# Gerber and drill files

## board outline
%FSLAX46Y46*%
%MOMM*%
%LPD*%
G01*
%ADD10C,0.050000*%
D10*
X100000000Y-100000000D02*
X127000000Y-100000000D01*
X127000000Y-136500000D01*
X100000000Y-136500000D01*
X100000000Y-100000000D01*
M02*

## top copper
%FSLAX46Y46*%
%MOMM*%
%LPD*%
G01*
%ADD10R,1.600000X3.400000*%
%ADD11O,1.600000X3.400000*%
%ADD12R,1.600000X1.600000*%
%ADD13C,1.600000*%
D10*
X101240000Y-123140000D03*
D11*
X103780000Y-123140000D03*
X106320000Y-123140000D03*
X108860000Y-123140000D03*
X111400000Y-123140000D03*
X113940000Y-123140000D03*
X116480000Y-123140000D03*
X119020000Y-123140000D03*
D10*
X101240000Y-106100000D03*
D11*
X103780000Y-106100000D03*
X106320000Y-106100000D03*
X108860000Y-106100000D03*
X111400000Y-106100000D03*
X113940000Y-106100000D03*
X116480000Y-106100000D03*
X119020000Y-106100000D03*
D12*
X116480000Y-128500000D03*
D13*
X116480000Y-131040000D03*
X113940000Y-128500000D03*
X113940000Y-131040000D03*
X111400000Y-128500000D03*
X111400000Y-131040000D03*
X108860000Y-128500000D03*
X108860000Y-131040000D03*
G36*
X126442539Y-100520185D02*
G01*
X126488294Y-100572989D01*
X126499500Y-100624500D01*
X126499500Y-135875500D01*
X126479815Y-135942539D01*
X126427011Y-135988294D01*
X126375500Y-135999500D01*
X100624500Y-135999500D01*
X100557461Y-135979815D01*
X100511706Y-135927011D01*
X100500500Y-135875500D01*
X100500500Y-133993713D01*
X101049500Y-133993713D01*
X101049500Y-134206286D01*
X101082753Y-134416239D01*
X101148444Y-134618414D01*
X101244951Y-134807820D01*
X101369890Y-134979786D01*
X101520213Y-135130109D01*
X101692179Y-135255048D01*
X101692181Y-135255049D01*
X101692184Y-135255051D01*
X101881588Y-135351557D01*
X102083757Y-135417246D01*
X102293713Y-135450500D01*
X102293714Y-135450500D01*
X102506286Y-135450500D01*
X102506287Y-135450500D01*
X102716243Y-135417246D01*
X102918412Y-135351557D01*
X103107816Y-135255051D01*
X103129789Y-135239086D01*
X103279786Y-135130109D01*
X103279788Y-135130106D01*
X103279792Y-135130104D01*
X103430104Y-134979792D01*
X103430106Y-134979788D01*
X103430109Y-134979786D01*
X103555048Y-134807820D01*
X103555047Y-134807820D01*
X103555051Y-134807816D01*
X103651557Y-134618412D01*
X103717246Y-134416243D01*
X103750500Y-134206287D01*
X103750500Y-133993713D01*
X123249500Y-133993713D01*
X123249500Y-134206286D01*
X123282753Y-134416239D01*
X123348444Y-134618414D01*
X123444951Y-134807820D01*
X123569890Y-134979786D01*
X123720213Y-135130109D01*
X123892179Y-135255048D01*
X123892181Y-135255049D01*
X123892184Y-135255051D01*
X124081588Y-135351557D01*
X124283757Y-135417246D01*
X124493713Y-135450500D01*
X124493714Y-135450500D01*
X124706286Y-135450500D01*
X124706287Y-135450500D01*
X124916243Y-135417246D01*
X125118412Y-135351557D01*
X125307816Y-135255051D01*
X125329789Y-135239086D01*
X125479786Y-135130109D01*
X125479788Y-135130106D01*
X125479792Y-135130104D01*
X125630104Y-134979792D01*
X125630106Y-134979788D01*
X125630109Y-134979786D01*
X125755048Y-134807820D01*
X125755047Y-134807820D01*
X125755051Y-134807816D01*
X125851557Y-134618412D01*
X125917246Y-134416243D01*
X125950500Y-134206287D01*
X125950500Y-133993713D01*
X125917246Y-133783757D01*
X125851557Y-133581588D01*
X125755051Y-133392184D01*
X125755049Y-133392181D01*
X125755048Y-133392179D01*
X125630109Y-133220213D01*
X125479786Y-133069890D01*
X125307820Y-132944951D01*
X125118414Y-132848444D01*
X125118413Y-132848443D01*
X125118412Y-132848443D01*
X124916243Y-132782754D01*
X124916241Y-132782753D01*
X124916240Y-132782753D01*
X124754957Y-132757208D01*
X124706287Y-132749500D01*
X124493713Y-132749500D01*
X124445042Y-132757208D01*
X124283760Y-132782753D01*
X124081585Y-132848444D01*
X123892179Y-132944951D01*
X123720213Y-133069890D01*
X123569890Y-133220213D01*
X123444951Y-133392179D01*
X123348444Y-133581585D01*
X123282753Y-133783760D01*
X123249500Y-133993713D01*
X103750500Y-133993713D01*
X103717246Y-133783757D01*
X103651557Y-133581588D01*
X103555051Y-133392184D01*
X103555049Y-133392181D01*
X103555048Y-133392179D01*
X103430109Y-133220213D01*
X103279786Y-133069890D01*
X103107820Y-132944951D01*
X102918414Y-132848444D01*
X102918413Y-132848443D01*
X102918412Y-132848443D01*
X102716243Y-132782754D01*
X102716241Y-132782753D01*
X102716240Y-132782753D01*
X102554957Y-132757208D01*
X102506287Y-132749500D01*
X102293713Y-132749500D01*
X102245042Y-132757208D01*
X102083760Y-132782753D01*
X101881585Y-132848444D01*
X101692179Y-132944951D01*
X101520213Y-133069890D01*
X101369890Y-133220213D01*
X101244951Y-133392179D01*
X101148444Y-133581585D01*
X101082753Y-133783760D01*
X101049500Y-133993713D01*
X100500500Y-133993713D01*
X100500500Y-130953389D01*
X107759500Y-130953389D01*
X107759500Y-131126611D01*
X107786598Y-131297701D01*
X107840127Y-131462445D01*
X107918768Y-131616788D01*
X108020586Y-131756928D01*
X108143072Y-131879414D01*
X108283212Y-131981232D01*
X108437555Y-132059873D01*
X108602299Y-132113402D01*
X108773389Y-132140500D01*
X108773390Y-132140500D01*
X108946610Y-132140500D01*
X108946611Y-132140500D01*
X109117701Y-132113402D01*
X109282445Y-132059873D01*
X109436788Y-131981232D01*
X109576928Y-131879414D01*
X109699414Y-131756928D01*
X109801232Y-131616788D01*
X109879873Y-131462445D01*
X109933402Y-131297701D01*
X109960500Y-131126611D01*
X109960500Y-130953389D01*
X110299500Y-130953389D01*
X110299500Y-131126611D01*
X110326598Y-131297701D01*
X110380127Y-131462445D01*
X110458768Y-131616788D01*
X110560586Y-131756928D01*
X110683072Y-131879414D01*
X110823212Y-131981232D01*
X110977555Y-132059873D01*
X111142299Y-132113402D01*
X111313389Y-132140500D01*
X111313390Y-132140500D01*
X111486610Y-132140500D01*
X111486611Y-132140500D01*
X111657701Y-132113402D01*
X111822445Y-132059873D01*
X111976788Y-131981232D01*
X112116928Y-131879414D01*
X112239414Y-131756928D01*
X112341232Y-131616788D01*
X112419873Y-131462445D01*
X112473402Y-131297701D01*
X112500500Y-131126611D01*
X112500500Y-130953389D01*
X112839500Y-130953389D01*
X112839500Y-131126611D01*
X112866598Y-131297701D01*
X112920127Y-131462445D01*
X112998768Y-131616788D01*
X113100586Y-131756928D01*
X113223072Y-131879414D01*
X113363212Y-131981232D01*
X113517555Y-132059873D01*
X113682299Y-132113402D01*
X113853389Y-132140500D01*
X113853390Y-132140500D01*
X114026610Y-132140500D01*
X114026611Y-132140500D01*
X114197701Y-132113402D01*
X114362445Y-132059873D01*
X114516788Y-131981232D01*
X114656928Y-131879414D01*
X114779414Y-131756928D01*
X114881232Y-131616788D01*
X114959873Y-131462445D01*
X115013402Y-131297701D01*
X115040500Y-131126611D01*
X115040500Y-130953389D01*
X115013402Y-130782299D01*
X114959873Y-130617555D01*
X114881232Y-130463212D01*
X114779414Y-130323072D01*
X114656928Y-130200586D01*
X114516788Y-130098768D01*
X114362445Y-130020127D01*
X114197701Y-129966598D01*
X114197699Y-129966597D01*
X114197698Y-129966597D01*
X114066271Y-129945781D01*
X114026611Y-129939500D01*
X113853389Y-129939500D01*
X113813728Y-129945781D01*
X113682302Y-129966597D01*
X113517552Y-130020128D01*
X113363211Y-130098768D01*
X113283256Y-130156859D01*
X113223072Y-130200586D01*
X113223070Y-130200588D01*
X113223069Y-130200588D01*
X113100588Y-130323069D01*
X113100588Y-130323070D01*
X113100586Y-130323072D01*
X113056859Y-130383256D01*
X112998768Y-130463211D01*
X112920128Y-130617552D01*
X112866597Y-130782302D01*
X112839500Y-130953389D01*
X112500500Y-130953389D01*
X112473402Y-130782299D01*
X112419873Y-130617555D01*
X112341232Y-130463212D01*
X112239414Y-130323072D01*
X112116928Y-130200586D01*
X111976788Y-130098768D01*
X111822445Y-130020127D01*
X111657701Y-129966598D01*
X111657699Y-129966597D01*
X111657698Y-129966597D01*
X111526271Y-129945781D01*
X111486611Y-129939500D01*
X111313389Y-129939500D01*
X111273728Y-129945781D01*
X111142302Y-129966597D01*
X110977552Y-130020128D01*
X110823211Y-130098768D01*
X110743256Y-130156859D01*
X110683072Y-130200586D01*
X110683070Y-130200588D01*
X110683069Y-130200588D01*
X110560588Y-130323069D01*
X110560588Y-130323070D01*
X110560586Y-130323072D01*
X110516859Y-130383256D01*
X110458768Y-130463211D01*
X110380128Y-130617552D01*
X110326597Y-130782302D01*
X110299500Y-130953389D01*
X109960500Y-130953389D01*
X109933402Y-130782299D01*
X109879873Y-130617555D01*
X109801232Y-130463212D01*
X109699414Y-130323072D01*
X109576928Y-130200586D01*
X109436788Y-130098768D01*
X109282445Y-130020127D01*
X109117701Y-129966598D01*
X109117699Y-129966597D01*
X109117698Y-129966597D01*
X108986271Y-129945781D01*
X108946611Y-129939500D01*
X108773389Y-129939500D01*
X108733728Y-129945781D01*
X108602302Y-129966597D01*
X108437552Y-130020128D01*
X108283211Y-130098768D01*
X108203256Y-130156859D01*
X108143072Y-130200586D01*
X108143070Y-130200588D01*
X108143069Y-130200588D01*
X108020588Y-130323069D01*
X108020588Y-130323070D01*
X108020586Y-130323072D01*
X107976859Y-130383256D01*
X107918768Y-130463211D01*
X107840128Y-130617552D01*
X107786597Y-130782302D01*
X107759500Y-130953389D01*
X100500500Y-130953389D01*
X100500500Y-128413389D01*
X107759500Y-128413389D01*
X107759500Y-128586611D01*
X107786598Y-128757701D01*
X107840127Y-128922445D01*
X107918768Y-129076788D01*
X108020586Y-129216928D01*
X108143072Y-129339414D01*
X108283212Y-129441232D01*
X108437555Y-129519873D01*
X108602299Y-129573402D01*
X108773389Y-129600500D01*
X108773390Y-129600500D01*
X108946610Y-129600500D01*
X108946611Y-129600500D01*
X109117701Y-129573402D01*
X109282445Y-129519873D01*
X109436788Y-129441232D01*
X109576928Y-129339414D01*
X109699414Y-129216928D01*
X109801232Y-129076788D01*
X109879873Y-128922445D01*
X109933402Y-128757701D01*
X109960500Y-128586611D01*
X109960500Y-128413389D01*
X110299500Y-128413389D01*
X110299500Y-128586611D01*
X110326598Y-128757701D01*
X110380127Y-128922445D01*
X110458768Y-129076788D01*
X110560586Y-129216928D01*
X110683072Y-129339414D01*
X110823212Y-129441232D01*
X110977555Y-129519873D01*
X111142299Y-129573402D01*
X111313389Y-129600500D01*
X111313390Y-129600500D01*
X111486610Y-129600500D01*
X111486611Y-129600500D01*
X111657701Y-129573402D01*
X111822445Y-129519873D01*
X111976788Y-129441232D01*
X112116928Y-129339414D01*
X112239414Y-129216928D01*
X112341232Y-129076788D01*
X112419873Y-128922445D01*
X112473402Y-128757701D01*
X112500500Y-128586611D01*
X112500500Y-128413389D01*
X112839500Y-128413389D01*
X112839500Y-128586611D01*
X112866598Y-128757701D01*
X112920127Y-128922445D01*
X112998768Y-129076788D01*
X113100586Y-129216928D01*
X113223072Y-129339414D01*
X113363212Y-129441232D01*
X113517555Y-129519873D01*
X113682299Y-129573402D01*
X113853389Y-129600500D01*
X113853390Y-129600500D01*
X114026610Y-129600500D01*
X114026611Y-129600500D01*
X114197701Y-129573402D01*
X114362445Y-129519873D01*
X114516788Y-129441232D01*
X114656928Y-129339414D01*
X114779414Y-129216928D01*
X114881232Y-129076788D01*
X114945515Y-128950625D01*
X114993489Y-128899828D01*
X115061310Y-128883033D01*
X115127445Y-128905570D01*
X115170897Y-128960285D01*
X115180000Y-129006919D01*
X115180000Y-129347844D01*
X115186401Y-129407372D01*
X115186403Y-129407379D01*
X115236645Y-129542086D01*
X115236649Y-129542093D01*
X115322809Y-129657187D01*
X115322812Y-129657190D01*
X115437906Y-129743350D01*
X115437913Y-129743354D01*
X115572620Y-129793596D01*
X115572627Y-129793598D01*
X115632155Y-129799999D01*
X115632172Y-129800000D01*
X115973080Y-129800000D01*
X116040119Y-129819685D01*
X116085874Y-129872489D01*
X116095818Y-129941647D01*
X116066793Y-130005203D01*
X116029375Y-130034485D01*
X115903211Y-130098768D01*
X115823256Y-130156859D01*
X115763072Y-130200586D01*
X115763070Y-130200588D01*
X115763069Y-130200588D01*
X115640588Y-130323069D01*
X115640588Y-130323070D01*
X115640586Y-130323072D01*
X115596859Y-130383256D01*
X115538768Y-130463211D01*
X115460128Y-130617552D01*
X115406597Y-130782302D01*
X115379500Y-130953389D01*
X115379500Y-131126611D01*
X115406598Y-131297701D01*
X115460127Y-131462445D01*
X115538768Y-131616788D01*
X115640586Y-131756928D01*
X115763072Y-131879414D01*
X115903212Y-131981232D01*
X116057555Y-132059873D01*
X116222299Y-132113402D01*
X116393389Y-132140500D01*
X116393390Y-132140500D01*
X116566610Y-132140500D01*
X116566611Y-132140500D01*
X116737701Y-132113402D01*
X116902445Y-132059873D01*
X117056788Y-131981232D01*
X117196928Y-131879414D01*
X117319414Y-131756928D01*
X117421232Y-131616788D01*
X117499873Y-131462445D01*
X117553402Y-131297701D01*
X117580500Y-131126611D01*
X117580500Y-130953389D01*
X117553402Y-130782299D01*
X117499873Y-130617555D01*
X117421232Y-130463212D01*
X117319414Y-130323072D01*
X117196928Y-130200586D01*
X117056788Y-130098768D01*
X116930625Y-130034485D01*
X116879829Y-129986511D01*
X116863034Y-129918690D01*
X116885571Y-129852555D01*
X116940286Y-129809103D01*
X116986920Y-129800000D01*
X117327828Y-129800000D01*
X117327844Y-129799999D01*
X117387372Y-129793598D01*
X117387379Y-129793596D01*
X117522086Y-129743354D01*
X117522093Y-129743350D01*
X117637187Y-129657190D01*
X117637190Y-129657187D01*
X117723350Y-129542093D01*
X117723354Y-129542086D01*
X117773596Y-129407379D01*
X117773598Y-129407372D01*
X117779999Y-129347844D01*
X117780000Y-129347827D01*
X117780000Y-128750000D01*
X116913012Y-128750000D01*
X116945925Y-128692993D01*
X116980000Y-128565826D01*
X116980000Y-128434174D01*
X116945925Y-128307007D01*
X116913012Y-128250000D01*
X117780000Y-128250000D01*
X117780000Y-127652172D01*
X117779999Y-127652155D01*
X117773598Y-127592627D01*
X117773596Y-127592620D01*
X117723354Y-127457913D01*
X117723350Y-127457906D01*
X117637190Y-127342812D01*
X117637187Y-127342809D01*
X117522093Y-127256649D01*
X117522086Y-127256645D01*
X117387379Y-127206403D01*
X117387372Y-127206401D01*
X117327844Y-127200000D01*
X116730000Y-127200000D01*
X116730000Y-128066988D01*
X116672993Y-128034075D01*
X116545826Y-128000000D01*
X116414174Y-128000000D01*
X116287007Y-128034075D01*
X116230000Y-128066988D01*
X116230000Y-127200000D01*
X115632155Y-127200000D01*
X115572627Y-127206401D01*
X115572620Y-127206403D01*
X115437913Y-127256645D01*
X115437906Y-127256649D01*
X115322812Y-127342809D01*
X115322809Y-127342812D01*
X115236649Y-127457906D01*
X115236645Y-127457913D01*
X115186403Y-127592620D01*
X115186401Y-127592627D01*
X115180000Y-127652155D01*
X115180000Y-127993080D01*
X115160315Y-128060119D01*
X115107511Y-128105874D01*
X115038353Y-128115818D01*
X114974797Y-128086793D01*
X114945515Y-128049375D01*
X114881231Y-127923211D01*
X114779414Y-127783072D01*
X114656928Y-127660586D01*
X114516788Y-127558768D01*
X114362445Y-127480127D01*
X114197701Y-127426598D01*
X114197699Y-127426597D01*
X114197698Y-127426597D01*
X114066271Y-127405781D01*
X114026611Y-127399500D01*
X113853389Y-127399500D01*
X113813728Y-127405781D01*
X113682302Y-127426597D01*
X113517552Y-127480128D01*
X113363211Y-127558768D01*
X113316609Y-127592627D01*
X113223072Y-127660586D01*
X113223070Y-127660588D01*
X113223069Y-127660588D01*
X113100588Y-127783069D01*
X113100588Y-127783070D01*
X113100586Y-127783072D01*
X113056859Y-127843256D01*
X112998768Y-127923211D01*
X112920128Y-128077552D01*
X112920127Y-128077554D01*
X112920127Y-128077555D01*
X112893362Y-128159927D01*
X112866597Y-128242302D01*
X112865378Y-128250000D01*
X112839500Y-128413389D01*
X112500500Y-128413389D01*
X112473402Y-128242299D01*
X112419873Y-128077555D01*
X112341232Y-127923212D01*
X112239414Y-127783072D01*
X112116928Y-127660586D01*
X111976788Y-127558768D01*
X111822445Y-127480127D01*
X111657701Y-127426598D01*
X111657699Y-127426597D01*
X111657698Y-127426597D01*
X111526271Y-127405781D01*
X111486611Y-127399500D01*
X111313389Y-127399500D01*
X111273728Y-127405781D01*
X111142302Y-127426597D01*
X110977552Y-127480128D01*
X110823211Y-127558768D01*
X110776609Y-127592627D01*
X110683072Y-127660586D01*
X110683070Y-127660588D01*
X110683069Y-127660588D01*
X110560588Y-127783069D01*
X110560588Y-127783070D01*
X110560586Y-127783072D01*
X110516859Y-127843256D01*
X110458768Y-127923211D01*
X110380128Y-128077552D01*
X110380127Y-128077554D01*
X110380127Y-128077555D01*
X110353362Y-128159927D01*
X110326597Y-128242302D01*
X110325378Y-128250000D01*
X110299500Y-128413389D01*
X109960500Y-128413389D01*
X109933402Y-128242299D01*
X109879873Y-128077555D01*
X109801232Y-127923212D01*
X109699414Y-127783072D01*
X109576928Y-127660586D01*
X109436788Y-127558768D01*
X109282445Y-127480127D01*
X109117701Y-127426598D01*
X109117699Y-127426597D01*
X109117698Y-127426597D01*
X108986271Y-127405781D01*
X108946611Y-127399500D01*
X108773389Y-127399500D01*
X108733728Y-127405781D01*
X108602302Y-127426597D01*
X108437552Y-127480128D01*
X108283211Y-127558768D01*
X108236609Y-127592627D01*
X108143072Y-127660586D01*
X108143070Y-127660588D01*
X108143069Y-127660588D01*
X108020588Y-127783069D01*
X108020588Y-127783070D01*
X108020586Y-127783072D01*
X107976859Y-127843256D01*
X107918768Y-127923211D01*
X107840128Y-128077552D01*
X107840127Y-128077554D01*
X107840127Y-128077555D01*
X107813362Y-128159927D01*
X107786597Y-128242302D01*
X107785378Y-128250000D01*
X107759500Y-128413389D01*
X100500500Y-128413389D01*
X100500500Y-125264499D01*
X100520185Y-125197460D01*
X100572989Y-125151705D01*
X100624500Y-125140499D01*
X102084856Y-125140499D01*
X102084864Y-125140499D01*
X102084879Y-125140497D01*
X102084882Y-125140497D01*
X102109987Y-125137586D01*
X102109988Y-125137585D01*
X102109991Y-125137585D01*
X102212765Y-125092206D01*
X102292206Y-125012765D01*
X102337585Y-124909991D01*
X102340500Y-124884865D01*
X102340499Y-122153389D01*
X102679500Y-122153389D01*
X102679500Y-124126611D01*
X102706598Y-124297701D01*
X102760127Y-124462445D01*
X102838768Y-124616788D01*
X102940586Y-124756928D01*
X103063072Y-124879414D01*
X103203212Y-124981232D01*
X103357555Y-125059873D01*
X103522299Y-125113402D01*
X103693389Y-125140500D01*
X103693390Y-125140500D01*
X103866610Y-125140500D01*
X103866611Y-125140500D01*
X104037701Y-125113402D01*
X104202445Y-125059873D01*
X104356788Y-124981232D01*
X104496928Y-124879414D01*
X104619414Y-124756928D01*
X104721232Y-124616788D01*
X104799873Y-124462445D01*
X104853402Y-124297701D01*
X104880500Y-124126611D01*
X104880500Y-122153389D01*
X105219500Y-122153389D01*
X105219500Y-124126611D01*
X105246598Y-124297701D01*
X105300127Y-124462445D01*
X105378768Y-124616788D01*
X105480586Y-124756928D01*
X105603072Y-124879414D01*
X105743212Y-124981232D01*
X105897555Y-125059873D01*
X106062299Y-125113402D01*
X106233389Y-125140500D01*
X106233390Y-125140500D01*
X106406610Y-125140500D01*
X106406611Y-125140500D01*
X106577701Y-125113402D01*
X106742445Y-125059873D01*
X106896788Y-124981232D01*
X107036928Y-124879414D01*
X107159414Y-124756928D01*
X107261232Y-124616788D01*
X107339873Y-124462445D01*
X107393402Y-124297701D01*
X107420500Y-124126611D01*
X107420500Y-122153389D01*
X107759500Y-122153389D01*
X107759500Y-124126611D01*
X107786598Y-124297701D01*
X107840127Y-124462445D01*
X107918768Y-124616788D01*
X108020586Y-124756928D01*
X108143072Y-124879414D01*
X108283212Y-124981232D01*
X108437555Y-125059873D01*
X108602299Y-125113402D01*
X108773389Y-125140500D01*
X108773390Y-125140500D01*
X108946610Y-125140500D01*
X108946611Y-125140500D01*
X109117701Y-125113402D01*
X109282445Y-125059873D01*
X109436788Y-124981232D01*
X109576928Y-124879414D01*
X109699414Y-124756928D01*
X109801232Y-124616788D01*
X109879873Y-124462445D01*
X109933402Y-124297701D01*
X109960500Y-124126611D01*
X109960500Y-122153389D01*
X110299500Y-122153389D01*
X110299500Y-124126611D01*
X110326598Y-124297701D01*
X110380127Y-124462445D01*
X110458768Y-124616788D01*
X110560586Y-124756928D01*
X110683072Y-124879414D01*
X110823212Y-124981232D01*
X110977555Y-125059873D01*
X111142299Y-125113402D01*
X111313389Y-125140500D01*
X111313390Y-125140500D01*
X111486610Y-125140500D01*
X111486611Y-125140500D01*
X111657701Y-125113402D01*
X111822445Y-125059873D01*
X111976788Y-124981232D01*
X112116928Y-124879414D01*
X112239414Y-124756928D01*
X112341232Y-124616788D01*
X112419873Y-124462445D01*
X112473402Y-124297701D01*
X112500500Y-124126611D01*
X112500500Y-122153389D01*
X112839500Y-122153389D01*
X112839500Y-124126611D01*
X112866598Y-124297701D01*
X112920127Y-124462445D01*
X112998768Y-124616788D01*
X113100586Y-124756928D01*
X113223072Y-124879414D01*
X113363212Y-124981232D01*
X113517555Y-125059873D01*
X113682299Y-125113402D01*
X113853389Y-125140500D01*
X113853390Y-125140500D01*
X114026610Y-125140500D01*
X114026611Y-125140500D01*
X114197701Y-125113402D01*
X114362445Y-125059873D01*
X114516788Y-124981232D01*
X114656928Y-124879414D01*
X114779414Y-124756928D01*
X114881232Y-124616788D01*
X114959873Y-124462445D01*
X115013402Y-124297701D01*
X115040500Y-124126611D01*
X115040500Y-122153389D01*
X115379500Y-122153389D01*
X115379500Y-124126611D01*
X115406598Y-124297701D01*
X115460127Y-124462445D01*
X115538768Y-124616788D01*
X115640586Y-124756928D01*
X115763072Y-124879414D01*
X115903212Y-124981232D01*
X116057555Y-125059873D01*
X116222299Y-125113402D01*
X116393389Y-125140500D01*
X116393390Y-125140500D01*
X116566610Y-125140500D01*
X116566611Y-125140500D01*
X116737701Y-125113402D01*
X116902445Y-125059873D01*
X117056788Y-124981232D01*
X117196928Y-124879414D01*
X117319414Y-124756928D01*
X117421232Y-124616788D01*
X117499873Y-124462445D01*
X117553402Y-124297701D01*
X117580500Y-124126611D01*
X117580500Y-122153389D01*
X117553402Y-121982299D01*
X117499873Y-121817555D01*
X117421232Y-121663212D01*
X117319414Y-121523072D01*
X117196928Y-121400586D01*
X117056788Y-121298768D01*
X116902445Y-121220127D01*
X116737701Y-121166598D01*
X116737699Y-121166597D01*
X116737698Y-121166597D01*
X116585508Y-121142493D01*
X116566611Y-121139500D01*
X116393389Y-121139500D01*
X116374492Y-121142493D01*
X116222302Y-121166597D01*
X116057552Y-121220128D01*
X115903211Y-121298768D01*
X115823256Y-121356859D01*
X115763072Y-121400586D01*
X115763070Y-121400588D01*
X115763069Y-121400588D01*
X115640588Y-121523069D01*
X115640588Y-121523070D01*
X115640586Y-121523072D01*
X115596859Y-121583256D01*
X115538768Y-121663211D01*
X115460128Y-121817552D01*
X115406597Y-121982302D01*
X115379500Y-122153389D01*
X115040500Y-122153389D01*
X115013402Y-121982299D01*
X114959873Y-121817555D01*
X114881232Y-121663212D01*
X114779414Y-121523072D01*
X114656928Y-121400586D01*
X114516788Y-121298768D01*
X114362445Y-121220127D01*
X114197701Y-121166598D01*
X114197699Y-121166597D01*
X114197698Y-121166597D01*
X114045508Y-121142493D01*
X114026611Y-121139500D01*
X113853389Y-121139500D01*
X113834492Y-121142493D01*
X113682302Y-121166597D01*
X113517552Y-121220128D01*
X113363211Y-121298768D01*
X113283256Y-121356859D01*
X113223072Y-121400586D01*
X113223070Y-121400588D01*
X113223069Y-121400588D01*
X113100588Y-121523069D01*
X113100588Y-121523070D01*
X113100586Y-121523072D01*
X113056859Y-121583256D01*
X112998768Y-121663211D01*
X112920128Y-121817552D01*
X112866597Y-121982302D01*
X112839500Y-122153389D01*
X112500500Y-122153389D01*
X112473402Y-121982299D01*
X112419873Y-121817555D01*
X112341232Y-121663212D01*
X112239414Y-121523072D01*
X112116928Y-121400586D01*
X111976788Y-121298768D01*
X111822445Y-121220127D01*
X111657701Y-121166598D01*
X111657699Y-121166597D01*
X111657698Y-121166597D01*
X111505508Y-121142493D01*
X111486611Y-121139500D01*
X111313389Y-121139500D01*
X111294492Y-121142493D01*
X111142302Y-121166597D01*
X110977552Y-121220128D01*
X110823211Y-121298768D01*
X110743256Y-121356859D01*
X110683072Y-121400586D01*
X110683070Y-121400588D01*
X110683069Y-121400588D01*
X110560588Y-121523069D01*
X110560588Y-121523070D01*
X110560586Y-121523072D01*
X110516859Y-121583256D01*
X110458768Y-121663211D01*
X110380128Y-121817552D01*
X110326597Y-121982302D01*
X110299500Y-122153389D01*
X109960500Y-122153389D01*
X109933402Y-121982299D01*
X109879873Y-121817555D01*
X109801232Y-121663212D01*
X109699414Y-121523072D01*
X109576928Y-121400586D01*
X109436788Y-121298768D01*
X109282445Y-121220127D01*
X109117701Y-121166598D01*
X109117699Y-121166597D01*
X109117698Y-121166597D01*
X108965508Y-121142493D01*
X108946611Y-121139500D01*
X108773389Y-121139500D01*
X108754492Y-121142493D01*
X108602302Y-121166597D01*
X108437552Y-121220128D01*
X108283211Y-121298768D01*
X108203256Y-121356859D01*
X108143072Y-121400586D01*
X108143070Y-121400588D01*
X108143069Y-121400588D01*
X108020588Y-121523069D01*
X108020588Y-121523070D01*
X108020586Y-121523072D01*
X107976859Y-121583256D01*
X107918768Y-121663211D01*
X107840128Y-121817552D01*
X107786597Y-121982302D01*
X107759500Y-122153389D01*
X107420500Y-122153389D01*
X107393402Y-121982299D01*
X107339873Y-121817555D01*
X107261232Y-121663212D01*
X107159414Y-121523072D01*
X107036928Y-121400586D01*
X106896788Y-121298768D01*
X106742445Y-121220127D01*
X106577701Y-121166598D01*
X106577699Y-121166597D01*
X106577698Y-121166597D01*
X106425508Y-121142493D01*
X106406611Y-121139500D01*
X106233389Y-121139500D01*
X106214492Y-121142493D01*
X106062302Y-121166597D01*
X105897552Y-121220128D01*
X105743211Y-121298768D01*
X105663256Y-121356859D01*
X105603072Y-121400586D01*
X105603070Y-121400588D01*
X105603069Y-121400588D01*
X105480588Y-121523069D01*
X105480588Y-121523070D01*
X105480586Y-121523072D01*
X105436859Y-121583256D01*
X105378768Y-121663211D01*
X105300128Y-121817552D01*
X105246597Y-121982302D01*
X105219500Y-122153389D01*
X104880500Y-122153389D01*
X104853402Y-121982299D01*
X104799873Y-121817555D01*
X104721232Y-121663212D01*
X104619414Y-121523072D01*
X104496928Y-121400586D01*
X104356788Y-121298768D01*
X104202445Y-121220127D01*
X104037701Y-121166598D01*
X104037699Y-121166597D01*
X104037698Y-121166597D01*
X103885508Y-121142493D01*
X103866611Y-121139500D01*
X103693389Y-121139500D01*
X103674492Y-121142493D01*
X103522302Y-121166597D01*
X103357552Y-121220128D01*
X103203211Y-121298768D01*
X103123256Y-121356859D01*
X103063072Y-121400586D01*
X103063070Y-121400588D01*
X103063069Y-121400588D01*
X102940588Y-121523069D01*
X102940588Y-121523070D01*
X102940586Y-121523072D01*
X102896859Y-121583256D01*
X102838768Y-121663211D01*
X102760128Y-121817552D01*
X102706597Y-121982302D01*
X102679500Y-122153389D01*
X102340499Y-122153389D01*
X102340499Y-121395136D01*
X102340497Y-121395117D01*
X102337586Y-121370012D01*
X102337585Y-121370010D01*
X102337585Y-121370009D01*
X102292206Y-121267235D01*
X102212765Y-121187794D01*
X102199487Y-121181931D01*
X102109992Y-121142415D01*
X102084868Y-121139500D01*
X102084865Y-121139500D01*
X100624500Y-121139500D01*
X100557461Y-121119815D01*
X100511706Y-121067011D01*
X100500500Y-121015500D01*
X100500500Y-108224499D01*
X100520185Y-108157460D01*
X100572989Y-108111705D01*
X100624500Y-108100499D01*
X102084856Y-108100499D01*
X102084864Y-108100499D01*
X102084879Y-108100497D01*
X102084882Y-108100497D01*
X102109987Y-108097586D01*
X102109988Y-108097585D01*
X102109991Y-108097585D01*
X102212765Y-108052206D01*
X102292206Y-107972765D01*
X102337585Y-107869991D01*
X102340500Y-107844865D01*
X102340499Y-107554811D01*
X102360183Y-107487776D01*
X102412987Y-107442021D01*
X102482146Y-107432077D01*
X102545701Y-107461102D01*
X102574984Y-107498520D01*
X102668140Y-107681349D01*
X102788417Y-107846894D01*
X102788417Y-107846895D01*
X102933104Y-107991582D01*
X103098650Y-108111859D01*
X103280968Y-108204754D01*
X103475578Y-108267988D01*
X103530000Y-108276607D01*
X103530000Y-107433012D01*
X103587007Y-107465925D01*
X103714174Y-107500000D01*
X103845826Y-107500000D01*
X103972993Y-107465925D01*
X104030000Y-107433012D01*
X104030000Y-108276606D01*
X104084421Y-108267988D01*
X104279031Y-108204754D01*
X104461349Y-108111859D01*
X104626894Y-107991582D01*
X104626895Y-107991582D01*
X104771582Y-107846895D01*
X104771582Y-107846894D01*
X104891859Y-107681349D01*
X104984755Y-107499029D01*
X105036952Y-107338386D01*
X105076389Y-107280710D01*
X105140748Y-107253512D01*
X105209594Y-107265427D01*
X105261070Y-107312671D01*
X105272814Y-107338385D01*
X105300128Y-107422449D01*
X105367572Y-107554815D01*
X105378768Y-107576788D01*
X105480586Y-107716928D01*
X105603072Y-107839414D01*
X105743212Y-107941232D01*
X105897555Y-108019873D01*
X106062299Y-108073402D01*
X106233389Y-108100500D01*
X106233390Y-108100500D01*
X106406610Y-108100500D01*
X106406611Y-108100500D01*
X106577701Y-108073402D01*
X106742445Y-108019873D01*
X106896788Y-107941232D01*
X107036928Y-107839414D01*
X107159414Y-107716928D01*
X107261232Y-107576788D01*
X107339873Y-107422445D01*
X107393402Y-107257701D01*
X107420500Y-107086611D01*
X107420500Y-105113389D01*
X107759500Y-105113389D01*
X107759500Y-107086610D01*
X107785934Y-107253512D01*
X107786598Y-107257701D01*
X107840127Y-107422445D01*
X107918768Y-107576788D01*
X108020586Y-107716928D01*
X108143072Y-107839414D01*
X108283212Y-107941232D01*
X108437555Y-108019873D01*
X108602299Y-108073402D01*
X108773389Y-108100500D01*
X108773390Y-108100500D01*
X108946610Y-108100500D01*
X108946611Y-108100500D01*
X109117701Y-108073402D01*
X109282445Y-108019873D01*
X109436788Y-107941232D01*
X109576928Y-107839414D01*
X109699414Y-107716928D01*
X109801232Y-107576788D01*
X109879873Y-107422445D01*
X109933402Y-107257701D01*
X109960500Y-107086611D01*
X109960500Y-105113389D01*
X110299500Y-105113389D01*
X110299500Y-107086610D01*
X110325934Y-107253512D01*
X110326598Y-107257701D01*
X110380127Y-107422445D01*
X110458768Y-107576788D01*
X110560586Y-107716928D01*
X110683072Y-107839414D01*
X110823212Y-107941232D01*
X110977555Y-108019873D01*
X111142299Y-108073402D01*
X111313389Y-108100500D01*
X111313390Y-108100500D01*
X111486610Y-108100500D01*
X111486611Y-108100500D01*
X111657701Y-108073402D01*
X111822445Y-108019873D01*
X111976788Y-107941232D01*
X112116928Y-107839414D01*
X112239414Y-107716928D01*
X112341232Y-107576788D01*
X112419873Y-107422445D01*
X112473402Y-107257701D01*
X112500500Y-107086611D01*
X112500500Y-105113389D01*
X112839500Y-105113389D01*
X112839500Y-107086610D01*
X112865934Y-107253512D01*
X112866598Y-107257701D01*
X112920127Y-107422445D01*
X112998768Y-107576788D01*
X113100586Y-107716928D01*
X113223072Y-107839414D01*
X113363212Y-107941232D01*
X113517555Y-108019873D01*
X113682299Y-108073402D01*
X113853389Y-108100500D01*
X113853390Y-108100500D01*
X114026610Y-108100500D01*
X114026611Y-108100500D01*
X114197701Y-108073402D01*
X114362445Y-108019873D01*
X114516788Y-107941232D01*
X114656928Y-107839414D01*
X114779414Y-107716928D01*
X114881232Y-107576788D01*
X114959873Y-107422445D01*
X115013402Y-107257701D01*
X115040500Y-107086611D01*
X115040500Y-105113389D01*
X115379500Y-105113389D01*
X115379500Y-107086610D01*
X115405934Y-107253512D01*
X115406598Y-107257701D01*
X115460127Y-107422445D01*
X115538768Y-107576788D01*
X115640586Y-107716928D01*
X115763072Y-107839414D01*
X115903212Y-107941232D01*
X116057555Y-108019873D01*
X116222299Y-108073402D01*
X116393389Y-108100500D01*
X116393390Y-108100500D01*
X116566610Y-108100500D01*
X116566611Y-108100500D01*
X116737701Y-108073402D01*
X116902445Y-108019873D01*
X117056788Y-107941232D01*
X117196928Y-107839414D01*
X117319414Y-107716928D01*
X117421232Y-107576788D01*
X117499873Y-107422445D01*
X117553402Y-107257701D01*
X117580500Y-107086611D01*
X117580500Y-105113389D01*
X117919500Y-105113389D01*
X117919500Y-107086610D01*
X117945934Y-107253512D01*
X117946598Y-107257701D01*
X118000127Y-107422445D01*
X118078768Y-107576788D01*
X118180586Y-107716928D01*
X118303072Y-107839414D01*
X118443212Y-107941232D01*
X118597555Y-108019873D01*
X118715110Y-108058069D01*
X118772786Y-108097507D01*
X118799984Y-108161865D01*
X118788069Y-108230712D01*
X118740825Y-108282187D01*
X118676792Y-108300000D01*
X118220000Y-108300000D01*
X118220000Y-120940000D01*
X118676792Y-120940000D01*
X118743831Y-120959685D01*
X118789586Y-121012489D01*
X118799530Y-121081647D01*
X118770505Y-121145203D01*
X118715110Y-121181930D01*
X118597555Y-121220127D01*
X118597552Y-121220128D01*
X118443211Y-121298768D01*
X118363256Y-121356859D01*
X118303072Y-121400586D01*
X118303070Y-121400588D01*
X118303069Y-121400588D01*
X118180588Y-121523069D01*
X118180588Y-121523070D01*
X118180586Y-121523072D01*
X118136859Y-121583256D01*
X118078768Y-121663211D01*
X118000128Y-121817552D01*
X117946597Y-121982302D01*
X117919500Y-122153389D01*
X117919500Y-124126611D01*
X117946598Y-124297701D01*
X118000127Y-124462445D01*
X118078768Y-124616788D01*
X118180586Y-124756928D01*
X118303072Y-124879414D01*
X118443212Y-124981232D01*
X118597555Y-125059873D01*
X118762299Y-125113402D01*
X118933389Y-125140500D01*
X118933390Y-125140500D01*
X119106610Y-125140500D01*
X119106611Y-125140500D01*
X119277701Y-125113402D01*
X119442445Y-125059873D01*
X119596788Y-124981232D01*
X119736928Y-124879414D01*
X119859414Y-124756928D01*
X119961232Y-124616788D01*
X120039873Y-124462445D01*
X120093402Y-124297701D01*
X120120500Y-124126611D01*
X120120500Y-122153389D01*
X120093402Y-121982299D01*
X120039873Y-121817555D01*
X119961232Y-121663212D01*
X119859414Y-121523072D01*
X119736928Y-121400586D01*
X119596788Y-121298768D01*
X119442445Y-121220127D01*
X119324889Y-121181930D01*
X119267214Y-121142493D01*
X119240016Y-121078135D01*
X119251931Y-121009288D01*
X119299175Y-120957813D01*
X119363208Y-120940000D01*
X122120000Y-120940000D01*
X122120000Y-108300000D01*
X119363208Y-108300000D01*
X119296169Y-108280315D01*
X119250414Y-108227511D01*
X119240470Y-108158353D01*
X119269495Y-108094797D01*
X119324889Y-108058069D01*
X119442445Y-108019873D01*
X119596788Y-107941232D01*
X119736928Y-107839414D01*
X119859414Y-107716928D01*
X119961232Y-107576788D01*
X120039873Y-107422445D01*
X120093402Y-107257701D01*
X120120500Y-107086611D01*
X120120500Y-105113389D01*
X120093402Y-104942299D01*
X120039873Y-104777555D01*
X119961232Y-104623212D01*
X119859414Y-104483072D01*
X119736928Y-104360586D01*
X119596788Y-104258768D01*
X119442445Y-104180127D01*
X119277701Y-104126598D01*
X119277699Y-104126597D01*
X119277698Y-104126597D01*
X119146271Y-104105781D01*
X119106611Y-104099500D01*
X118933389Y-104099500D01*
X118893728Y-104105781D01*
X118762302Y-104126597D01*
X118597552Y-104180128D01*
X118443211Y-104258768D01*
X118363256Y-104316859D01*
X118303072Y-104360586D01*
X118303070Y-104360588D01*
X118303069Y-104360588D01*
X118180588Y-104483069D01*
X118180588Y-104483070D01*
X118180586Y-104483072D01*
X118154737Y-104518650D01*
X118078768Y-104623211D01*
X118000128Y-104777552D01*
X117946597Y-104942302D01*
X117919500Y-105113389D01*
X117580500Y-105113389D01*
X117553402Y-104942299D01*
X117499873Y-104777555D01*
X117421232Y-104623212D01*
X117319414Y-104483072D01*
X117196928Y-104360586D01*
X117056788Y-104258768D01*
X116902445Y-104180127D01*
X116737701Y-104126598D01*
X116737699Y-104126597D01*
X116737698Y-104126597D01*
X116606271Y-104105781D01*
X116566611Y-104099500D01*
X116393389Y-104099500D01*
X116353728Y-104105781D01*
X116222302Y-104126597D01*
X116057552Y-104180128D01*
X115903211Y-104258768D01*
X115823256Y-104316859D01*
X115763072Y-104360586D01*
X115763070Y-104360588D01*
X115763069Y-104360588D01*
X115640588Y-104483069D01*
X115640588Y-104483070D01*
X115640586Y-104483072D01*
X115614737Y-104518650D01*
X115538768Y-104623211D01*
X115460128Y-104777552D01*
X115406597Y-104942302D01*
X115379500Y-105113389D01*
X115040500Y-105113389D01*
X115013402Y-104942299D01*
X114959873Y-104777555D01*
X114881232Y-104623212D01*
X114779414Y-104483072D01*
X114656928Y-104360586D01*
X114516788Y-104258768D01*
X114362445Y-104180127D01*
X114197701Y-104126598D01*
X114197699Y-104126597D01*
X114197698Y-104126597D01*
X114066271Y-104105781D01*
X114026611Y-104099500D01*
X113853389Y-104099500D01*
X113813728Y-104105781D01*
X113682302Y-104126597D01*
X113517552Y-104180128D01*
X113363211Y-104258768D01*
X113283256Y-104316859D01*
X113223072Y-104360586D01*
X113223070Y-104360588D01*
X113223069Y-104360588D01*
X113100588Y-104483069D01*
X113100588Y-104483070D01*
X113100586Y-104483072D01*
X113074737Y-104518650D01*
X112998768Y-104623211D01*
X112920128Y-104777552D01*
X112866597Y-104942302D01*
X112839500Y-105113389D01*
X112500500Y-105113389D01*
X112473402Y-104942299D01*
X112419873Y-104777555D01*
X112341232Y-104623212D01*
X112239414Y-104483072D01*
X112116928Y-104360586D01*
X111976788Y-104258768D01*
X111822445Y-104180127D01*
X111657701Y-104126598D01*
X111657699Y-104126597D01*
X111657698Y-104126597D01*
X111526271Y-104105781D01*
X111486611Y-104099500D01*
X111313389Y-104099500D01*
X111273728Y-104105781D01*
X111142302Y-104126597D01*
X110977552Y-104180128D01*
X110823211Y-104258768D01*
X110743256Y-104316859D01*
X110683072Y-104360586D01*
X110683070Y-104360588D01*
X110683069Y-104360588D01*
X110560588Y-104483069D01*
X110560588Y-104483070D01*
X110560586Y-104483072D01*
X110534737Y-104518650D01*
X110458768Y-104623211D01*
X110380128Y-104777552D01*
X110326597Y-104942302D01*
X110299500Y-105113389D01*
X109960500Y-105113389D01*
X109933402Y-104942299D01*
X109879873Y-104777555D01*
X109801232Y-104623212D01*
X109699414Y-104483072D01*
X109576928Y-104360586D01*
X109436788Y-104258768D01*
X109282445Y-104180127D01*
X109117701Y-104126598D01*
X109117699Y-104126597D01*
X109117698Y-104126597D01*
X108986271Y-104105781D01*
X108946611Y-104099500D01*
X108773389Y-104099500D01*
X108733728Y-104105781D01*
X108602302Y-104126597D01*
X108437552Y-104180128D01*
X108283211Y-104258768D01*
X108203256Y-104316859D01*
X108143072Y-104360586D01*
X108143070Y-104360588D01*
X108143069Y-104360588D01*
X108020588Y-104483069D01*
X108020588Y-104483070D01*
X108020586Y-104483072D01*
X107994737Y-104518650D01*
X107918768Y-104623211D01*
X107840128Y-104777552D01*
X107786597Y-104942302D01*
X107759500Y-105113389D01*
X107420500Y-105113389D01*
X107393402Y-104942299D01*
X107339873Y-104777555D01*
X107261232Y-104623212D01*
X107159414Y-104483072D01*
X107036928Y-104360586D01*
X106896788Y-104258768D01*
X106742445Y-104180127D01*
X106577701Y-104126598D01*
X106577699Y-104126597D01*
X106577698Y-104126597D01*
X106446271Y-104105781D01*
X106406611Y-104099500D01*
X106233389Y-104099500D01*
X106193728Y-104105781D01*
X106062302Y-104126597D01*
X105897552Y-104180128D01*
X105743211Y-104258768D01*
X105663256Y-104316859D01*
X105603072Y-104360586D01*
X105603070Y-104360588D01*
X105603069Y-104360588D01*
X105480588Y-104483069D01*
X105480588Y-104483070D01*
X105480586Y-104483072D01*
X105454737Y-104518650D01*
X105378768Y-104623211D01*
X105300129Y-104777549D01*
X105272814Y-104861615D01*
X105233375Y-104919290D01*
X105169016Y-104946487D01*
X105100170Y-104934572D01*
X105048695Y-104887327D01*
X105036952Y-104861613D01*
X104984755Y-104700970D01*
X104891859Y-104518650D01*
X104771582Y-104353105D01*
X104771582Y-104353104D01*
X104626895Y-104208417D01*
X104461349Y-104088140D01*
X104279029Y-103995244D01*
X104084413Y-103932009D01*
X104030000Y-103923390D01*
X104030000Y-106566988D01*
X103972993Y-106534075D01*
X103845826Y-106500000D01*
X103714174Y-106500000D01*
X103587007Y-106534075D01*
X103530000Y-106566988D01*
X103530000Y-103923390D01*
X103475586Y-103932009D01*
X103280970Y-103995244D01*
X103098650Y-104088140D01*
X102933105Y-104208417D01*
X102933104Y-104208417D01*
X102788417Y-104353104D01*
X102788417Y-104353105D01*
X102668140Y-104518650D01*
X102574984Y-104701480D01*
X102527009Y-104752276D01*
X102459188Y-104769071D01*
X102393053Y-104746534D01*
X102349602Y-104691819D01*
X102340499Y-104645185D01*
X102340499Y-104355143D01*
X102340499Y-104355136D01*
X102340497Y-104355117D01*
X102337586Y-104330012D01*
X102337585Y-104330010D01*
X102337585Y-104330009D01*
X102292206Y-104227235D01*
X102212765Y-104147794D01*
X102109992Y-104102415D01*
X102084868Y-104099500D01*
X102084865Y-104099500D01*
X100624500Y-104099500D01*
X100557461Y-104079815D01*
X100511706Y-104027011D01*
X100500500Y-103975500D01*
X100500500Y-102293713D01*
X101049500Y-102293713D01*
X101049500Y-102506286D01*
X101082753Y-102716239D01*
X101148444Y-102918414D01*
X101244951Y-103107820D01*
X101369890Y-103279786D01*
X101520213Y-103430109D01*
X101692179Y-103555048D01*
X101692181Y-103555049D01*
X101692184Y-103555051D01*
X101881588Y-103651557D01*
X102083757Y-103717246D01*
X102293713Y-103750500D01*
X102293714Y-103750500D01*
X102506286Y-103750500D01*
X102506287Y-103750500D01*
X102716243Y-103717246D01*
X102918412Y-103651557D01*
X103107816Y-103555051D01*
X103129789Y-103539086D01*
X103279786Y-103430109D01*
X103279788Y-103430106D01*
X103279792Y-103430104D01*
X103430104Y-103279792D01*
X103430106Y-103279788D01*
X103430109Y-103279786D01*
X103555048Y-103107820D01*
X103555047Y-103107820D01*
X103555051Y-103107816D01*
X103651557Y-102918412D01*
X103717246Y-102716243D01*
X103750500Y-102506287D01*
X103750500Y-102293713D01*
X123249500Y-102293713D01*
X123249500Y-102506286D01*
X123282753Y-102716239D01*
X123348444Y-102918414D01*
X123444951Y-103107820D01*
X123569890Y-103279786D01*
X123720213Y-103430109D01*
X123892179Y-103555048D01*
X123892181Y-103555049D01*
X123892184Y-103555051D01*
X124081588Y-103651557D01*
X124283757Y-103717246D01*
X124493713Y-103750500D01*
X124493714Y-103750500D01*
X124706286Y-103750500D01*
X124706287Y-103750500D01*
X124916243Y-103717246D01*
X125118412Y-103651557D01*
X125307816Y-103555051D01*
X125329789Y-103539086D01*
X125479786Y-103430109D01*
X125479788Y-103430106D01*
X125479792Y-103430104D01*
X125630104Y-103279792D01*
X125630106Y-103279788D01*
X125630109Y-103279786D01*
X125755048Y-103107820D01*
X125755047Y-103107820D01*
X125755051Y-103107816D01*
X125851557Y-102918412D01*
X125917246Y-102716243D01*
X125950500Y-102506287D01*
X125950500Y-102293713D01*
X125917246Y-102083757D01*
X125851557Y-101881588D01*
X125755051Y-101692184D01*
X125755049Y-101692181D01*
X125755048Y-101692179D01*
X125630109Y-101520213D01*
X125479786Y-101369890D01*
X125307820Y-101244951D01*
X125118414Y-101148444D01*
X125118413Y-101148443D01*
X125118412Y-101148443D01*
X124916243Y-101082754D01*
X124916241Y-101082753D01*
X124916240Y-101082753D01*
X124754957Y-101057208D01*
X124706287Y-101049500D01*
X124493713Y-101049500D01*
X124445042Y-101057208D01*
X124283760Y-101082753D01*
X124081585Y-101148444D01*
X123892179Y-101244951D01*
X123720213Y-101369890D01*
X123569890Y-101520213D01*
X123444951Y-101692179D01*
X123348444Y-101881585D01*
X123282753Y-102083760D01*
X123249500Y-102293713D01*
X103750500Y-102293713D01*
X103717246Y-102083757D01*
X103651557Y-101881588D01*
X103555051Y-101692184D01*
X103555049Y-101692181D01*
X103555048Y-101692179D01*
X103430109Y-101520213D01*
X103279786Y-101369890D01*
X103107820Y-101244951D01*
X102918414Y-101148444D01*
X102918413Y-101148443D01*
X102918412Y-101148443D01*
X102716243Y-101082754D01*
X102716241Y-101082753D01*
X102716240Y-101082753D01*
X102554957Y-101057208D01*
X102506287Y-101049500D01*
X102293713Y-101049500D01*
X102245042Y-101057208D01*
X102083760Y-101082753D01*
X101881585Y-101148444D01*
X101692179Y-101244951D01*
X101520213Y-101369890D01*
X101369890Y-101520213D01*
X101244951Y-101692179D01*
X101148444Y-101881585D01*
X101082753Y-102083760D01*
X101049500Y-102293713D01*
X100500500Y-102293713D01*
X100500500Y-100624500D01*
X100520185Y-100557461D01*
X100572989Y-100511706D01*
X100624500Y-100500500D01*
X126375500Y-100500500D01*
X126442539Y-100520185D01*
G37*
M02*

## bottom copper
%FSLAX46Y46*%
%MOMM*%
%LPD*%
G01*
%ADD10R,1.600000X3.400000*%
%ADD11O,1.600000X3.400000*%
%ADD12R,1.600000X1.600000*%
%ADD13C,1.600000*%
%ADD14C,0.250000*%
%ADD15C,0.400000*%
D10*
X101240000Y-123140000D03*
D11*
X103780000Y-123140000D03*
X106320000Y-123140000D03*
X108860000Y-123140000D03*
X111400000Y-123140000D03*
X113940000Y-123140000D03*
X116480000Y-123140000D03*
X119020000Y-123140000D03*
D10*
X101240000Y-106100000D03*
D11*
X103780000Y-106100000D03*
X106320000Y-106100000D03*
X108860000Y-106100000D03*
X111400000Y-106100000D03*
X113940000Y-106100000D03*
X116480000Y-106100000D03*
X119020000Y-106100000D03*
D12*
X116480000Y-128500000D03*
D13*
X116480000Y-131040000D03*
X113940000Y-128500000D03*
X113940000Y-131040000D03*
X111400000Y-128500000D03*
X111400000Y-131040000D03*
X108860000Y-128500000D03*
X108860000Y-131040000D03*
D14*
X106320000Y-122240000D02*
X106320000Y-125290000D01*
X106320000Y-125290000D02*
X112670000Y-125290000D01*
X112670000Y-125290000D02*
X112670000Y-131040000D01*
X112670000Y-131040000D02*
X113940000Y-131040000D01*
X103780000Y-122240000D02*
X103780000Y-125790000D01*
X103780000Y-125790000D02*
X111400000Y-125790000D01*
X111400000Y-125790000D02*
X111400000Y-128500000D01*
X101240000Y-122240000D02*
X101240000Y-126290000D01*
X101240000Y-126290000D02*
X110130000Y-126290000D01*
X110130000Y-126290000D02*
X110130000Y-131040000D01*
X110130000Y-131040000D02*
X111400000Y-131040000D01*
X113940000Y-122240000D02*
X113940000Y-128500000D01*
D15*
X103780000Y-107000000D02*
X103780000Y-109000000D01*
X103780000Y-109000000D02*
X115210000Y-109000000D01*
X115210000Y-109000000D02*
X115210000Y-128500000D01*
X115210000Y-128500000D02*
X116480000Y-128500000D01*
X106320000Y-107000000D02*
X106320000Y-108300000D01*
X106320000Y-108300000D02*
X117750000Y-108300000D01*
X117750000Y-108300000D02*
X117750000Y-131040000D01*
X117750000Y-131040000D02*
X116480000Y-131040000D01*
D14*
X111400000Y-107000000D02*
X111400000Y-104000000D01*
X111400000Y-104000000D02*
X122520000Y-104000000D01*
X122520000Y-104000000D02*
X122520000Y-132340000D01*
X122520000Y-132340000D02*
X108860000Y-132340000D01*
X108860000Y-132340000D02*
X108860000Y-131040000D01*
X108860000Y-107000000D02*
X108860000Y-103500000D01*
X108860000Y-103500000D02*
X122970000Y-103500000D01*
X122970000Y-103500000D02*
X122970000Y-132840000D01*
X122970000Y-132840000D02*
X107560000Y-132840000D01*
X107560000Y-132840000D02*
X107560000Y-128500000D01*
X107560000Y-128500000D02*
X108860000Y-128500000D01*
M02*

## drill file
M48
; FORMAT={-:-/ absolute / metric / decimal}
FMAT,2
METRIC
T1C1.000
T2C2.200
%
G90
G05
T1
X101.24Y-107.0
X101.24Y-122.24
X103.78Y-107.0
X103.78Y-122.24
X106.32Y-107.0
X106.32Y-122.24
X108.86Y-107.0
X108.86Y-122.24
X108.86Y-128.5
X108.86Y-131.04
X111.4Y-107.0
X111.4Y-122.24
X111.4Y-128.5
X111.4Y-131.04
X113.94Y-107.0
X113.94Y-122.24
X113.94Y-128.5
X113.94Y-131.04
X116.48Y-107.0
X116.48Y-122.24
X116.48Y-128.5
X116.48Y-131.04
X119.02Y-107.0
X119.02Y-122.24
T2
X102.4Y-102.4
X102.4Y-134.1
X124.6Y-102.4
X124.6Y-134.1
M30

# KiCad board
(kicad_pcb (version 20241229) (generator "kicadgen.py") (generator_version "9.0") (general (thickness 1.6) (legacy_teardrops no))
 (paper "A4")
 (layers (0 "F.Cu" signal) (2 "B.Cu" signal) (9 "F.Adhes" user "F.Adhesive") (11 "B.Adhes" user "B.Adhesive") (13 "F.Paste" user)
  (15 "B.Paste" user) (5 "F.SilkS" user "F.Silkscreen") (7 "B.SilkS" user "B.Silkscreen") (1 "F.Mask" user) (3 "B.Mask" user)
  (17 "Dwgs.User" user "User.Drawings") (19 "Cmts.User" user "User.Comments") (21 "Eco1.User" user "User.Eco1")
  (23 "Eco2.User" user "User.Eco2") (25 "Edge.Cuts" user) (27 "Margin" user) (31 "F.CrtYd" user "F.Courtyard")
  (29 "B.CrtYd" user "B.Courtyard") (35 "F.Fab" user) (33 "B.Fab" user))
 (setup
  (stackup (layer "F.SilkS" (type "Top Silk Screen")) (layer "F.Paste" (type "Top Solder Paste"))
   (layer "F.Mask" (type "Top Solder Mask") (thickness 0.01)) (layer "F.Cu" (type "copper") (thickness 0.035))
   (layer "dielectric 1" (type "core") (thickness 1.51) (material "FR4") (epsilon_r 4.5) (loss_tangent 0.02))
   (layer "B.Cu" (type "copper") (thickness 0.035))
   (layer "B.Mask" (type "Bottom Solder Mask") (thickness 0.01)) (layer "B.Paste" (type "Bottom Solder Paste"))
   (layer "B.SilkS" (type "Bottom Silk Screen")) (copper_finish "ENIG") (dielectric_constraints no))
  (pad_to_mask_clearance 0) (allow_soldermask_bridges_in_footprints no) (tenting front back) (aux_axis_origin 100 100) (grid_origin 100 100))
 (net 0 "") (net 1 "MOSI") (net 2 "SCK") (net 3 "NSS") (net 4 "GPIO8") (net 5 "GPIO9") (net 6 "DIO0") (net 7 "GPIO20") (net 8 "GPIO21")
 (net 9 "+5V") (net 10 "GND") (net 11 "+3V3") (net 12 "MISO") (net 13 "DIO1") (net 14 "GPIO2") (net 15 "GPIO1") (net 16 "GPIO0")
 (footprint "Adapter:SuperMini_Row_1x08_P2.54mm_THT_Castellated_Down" (layer "F.Cu") (at 101.24 122.24)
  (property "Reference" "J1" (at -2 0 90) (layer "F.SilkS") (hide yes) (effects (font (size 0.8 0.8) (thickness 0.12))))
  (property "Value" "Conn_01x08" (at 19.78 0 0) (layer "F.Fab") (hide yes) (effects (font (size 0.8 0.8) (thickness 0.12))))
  (pad "1" thru_hole rect (at 0 0) (size 1.6 3.4) (drill 1 (offset 0 0.9)) (layers "*.Cu" "*.Mask") (remove_unused_layers no) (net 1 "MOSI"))
  (pad "2" thru_hole oval (at 2.54 0) (size 1.6 3.4) (drill 1 (offset 0 0.9)) (layers "*.Cu" "*.Mask") (remove_unused_layers no)
   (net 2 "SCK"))
  (pad "3" thru_hole oval (at 5.08 0) (size 1.6 3.4) (drill 1 (offset 0 0.9)) (layers "*.Cu" "*.Mask") (remove_unused_layers no)
   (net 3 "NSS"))
  (pad "4" thru_hole oval (at 7.62 0) (size 1.6 3.4) (drill 1 (offset 0 0.9)) (layers "*.Cu" "*.Mask") (remove_unused_layers no)
   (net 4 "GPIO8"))
  (pad "5" thru_hole oval (at 10.16 0) (size 1.6 3.4) (drill 1 (offset 0 0.9)) (layers "*.Cu" "*.Mask") (remove_unused_layers no)
   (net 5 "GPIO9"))
  (pad "6" thru_hole oval (at 12.7 0) (size 1.6 3.4) (drill 1 (offset 0 0.9)) (layers "*.Cu" "*.Mask") (remove_unused_layers no)
   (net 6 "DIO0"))
  (pad "7" thru_hole oval (at 15.24 0) (size 1.6 3.4) (drill 1 (offset 0 0.9)) (layers "*.Cu" "*.Mask") (remove_unused_layers no)
   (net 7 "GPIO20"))
  (pad "8" thru_hole oval (at 17.78 0) (size 1.6 3.4) (drill 1 (offset 0 0.9)) (layers "*.Cu" "*.Mask") (remove_unused_layers no)
   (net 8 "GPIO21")))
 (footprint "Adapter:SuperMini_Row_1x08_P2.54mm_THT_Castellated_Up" (layer "F.Cu") (at 101.24 107)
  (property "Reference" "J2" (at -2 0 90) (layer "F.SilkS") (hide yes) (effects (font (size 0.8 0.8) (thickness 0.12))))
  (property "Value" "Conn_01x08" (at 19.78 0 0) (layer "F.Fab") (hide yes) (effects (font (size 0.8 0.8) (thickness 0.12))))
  (pad "1" thru_hole rect (at 0 0) (size 1.6 3.4) (drill 1 (offset 0 -0.9)) (layers "*.Cu" "*.Mask") (remove_unused_layers no) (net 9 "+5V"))
  (pad "2" thru_hole oval (at 2.54 0) (size 1.6 3.4) (drill 1 (offset 0 -0.9)) (layers "*.Cu" "*.Mask") (remove_unused_layers no)
   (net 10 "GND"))
  (pad "3" thru_hole oval (at 5.08 0) (size 1.6 3.4) (drill 1 (offset 0 -0.9)) (layers "*.Cu" "*.Mask") (remove_unused_layers no)
   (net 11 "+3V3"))
  (pad "4" thru_hole oval (at 7.62 0) (size 1.6 3.4) (drill 1 (offset 0 -0.9)) (layers "*.Cu" "*.Mask") (remove_unused_layers no)
   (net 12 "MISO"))
  (pad "5" thru_hole oval (at 10.16 0) (size 1.6 3.4) (drill 1 (offset 0 -0.9)) (layers "*.Cu" "*.Mask") (remove_unused_layers no)
   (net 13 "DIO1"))
  (pad "6" thru_hole oval (at 12.7 0) (size 1.6 3.4) (drill 1 (offset 0 -0.9)) (layers "*.Cu" "*.Mask") (remove_unused_layers no)
   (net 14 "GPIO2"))
  (pad "7" thru_hole oval (at 15.24 0) (size 1.6 3.4) (drill 1 (offset 0 -0.9)) (layers "*.Cu" "*.Mask") (remove_unused_layers no)
   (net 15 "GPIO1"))
  (pad "8" thru_hole oval (at 17.78 0) (size 1.6 3.4) (drill 1 (offset 0 -0.9)) (layers "*.Cu" "*.Mask") (remove_unused_layers no)
   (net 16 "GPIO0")))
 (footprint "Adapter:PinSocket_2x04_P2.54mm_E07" (layer "F.Cu") (at 116.48 128.5)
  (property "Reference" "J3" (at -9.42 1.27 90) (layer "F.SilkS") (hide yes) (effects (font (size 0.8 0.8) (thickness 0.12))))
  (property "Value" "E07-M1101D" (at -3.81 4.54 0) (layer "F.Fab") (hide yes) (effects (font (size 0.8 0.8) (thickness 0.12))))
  (pad "1" thru_hole rect (at 0 0) (size 1.6 1.6) (drill 1) (layers "*.Cu" "*.Mask") (remove_unused_layers no) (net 10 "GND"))
  (pad "2" thru_hole circle (at 0 2.54) (size 1.6 1.6) (drill 1) (layers "*.Cu" "*.Mask") (remove_unused_layers no) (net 11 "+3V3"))
  (pad "3" thru_hole circle (at -2.54 0) (size 1.6 1.6) (drill 1) (layers "*.Cu" "*.Mask") (remove_unused_layers no) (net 6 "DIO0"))
  (pad "4" thru_hole circle (at -2.54 2.54) (size 1.6 1.6) (drill 1) (layers "*.Cu" "*.Mask") (remove_unused_layers no) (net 3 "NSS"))
  (pad "5" thru_hole circle (at -5.08 0) (size 1.6 1.6) (drill 1) (layers "*.Cu" "*.Mask") (remove_unused_layers no) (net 2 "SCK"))
  (pad "6" thru_hole circle (at -5.08 2.54) (size 1.6 1.6) (drill 1) (layers "*.Cu" "*.Mask") (remove_unused_layers no) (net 1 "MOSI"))
  (pad "7" thru_hole circle (at -7.62 0) (size 1.6 1.6) (drill 1) (layers "*.Cu" "*.Mask") (remove_unused_layers no) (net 12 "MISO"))
  (pad "8" thru_hole circle (at -7.62 2.54) (size 1.6 1.6) (drill 1) (layers "*.Cu" "*.Mask") (remove_unused_layers no) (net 13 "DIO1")))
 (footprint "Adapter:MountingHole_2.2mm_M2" (layer "F.Cu") (at 102.4 102.4)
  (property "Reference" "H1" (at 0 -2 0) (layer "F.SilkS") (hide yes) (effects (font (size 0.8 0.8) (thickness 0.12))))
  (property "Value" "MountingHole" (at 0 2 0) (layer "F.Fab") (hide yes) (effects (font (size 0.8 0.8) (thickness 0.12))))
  (pad "1" np_thru_hole circle (at 0 0) (size 2.2 2.2) (drill 2.2) (layers "*.Cu" "*.Mask")))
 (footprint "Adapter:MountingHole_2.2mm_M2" (layer "F.Cu") (at 124.6 102.4)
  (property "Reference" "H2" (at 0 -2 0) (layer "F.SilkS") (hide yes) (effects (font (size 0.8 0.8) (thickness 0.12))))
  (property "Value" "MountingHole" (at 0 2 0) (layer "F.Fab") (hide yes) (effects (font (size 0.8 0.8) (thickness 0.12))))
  (pad "1" np_thru_hole circle (at 0 0) (size 2.2 2.2) (drill 2.2) (layers "*.Cu" "*.Mask")))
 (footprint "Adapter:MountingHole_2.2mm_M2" (layer "F.Cu") (at 102.4 134.1)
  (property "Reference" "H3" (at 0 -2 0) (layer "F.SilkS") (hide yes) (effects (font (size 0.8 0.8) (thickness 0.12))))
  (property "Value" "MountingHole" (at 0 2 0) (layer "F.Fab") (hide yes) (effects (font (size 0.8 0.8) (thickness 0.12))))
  (pad "1" np_thru_hole circle (at 0 0) (size 2.2 2.2) (drill 2.2) (layers "*.Cu" "*.Mask")))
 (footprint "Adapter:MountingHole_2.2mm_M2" (layer "F.Cu") (at 124.6 134.1)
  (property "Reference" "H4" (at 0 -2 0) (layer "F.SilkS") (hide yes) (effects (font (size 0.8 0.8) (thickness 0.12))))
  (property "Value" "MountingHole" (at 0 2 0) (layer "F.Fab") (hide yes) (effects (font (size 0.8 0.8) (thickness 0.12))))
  (pad "1" np_thru_hole circle (at 0 0) (size 2.2 2.2) (drill 2.2) (layers "*.Cu" "*.Mask")))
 (gr_rect (start 100 100) (end 127 136.5) (stroke (width 0.05) (type solid)) (fill no) (layer "Edge.Cuts"))
 (segment (start 106.32 122.24) (end 106.32 125.29) (width 0.25) (layer "B.Cu") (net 3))
 (segment (start 106.32 125.29) (end 112.67 125.29) (width 0.25) (layer "B.Cu") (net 3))
 (segment (start 112.67 125.29) (end 112.67 131.04) (width 0.25) (layer "B.Cu") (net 3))
 (segment (start 112.67 131.04) (end 113.94 131.04) (width 0.25) (layer "B.Cu") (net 3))
 (segment (start 103.78 122.24) (end 103.78 125.79) (width 0.25) (layer "B.Cu") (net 2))
 (segment (start 103.78 125.79) (end 111.4 125.79) (width 0.25) (layer "B.Cu") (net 2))
 (segment (start 111.4 125.79) (end 111.4 128.5) (width 0.25) (layer "B.Cu") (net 2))
 (segment (start 101.24 122.24) (end 101.24 126.29) (width 0.25) (layer "B.Cu") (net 1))
 (segment (start 101.24 126.29) (end 110.13 126.29) (width 0.25) (layer "B.Cu") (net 1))
 (segment (start 110.13 126.29) (end 110.13 131.04) (width 0.25) (layer "B.Cu") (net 1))
 (segment (start 110.13 131.04) (end 111.4 131.04) (width 0.25) (layer "B.Cu") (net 1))
 (segment (start 113.94 122.24) (end 113.94 128.5) (width 0.25) (layer "B.Cu") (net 6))
 (segment (start 103.78 107) (end 103.78 109) (width 0.4) (layer "B.Cu") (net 10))
 (segment (start 103.78 109) (end 115.21 109) (width 0.4) (layer "B.Cu") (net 10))
 (segment (start 115.21 109) (end 115.21 128.5) (width 0.4) (layer "B.Cu") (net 10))
 (segment (start 115.21 128.5) (end 116.48 128.5) (width 0.4) (layer "B.Cu") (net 10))
 (segment (start 106.32 107) (end 106.32 108.3) (width 0.4) (layer "B.Cu") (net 11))
 (segment (start 106.32 108.3) (end 117.75 108.3) (width 0.4) (layer "B.Cu") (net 11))
 (segment (start 117.75 108.3) (end 117.75 131.04) (width 0.4) (layer "B.Cu") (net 11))
 (segment (start 117.75 131.04) (end 116.48 131.04) (width 0.4) (layer "B.Cu") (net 11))
 (segment (start 111.4 107) (end 111.4 104) (width 0.25) (layer "B.Cu") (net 13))
 (segment (start 111.4 104) (end 122.52 104) (width 0.25) (layer "B.Cu") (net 13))
 (segment (start 122.52 104) (end 122.52 132.34) (width 0.25) (layer "B.Cu") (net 13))
 (segment (start 122.52 132.34) (end 108.86 132.34) (width 0.25) (layer "B.Cu") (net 13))
 (segment (start 108.86 132.34) (end 108.86 131.04) (width 0.25) (layer "B.Cu") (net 13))
 (segment (start 108.86 107) (end 108.86 103.5) (width 0.25) (layer "B.Cu") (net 12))
 (segment (start 108.86 103.5) (end 122.97 103.5) (width 0.25) (layer "B.Cu") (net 12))
 (segment (start 122.97 103.5) (end 122.97 132.84) (width 0.25) (layer "B.Cu") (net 12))
 (segment (start 122.97 132.84) (end 107.56 132.84) (width 0.25) (layer "B.Cu") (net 12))
 (segment (start 107.56 132.84) (end 107.56 128.5) (width 0.25) (layer "B.Cu") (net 12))
 (segment (start 107.56 128.5) (end 108.86 128.5) (width 0.25) (layer "B.Cu") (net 12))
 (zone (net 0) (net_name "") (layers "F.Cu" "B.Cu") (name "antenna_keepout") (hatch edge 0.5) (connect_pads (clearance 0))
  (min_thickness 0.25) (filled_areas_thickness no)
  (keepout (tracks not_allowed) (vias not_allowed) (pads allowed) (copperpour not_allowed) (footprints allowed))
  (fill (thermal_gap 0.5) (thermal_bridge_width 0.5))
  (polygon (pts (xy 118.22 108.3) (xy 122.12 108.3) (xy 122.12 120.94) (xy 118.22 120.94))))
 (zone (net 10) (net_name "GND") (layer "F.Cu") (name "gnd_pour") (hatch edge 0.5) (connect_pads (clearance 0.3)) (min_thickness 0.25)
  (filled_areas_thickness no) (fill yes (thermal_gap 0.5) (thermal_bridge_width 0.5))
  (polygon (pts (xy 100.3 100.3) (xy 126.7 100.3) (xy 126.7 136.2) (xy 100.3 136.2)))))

